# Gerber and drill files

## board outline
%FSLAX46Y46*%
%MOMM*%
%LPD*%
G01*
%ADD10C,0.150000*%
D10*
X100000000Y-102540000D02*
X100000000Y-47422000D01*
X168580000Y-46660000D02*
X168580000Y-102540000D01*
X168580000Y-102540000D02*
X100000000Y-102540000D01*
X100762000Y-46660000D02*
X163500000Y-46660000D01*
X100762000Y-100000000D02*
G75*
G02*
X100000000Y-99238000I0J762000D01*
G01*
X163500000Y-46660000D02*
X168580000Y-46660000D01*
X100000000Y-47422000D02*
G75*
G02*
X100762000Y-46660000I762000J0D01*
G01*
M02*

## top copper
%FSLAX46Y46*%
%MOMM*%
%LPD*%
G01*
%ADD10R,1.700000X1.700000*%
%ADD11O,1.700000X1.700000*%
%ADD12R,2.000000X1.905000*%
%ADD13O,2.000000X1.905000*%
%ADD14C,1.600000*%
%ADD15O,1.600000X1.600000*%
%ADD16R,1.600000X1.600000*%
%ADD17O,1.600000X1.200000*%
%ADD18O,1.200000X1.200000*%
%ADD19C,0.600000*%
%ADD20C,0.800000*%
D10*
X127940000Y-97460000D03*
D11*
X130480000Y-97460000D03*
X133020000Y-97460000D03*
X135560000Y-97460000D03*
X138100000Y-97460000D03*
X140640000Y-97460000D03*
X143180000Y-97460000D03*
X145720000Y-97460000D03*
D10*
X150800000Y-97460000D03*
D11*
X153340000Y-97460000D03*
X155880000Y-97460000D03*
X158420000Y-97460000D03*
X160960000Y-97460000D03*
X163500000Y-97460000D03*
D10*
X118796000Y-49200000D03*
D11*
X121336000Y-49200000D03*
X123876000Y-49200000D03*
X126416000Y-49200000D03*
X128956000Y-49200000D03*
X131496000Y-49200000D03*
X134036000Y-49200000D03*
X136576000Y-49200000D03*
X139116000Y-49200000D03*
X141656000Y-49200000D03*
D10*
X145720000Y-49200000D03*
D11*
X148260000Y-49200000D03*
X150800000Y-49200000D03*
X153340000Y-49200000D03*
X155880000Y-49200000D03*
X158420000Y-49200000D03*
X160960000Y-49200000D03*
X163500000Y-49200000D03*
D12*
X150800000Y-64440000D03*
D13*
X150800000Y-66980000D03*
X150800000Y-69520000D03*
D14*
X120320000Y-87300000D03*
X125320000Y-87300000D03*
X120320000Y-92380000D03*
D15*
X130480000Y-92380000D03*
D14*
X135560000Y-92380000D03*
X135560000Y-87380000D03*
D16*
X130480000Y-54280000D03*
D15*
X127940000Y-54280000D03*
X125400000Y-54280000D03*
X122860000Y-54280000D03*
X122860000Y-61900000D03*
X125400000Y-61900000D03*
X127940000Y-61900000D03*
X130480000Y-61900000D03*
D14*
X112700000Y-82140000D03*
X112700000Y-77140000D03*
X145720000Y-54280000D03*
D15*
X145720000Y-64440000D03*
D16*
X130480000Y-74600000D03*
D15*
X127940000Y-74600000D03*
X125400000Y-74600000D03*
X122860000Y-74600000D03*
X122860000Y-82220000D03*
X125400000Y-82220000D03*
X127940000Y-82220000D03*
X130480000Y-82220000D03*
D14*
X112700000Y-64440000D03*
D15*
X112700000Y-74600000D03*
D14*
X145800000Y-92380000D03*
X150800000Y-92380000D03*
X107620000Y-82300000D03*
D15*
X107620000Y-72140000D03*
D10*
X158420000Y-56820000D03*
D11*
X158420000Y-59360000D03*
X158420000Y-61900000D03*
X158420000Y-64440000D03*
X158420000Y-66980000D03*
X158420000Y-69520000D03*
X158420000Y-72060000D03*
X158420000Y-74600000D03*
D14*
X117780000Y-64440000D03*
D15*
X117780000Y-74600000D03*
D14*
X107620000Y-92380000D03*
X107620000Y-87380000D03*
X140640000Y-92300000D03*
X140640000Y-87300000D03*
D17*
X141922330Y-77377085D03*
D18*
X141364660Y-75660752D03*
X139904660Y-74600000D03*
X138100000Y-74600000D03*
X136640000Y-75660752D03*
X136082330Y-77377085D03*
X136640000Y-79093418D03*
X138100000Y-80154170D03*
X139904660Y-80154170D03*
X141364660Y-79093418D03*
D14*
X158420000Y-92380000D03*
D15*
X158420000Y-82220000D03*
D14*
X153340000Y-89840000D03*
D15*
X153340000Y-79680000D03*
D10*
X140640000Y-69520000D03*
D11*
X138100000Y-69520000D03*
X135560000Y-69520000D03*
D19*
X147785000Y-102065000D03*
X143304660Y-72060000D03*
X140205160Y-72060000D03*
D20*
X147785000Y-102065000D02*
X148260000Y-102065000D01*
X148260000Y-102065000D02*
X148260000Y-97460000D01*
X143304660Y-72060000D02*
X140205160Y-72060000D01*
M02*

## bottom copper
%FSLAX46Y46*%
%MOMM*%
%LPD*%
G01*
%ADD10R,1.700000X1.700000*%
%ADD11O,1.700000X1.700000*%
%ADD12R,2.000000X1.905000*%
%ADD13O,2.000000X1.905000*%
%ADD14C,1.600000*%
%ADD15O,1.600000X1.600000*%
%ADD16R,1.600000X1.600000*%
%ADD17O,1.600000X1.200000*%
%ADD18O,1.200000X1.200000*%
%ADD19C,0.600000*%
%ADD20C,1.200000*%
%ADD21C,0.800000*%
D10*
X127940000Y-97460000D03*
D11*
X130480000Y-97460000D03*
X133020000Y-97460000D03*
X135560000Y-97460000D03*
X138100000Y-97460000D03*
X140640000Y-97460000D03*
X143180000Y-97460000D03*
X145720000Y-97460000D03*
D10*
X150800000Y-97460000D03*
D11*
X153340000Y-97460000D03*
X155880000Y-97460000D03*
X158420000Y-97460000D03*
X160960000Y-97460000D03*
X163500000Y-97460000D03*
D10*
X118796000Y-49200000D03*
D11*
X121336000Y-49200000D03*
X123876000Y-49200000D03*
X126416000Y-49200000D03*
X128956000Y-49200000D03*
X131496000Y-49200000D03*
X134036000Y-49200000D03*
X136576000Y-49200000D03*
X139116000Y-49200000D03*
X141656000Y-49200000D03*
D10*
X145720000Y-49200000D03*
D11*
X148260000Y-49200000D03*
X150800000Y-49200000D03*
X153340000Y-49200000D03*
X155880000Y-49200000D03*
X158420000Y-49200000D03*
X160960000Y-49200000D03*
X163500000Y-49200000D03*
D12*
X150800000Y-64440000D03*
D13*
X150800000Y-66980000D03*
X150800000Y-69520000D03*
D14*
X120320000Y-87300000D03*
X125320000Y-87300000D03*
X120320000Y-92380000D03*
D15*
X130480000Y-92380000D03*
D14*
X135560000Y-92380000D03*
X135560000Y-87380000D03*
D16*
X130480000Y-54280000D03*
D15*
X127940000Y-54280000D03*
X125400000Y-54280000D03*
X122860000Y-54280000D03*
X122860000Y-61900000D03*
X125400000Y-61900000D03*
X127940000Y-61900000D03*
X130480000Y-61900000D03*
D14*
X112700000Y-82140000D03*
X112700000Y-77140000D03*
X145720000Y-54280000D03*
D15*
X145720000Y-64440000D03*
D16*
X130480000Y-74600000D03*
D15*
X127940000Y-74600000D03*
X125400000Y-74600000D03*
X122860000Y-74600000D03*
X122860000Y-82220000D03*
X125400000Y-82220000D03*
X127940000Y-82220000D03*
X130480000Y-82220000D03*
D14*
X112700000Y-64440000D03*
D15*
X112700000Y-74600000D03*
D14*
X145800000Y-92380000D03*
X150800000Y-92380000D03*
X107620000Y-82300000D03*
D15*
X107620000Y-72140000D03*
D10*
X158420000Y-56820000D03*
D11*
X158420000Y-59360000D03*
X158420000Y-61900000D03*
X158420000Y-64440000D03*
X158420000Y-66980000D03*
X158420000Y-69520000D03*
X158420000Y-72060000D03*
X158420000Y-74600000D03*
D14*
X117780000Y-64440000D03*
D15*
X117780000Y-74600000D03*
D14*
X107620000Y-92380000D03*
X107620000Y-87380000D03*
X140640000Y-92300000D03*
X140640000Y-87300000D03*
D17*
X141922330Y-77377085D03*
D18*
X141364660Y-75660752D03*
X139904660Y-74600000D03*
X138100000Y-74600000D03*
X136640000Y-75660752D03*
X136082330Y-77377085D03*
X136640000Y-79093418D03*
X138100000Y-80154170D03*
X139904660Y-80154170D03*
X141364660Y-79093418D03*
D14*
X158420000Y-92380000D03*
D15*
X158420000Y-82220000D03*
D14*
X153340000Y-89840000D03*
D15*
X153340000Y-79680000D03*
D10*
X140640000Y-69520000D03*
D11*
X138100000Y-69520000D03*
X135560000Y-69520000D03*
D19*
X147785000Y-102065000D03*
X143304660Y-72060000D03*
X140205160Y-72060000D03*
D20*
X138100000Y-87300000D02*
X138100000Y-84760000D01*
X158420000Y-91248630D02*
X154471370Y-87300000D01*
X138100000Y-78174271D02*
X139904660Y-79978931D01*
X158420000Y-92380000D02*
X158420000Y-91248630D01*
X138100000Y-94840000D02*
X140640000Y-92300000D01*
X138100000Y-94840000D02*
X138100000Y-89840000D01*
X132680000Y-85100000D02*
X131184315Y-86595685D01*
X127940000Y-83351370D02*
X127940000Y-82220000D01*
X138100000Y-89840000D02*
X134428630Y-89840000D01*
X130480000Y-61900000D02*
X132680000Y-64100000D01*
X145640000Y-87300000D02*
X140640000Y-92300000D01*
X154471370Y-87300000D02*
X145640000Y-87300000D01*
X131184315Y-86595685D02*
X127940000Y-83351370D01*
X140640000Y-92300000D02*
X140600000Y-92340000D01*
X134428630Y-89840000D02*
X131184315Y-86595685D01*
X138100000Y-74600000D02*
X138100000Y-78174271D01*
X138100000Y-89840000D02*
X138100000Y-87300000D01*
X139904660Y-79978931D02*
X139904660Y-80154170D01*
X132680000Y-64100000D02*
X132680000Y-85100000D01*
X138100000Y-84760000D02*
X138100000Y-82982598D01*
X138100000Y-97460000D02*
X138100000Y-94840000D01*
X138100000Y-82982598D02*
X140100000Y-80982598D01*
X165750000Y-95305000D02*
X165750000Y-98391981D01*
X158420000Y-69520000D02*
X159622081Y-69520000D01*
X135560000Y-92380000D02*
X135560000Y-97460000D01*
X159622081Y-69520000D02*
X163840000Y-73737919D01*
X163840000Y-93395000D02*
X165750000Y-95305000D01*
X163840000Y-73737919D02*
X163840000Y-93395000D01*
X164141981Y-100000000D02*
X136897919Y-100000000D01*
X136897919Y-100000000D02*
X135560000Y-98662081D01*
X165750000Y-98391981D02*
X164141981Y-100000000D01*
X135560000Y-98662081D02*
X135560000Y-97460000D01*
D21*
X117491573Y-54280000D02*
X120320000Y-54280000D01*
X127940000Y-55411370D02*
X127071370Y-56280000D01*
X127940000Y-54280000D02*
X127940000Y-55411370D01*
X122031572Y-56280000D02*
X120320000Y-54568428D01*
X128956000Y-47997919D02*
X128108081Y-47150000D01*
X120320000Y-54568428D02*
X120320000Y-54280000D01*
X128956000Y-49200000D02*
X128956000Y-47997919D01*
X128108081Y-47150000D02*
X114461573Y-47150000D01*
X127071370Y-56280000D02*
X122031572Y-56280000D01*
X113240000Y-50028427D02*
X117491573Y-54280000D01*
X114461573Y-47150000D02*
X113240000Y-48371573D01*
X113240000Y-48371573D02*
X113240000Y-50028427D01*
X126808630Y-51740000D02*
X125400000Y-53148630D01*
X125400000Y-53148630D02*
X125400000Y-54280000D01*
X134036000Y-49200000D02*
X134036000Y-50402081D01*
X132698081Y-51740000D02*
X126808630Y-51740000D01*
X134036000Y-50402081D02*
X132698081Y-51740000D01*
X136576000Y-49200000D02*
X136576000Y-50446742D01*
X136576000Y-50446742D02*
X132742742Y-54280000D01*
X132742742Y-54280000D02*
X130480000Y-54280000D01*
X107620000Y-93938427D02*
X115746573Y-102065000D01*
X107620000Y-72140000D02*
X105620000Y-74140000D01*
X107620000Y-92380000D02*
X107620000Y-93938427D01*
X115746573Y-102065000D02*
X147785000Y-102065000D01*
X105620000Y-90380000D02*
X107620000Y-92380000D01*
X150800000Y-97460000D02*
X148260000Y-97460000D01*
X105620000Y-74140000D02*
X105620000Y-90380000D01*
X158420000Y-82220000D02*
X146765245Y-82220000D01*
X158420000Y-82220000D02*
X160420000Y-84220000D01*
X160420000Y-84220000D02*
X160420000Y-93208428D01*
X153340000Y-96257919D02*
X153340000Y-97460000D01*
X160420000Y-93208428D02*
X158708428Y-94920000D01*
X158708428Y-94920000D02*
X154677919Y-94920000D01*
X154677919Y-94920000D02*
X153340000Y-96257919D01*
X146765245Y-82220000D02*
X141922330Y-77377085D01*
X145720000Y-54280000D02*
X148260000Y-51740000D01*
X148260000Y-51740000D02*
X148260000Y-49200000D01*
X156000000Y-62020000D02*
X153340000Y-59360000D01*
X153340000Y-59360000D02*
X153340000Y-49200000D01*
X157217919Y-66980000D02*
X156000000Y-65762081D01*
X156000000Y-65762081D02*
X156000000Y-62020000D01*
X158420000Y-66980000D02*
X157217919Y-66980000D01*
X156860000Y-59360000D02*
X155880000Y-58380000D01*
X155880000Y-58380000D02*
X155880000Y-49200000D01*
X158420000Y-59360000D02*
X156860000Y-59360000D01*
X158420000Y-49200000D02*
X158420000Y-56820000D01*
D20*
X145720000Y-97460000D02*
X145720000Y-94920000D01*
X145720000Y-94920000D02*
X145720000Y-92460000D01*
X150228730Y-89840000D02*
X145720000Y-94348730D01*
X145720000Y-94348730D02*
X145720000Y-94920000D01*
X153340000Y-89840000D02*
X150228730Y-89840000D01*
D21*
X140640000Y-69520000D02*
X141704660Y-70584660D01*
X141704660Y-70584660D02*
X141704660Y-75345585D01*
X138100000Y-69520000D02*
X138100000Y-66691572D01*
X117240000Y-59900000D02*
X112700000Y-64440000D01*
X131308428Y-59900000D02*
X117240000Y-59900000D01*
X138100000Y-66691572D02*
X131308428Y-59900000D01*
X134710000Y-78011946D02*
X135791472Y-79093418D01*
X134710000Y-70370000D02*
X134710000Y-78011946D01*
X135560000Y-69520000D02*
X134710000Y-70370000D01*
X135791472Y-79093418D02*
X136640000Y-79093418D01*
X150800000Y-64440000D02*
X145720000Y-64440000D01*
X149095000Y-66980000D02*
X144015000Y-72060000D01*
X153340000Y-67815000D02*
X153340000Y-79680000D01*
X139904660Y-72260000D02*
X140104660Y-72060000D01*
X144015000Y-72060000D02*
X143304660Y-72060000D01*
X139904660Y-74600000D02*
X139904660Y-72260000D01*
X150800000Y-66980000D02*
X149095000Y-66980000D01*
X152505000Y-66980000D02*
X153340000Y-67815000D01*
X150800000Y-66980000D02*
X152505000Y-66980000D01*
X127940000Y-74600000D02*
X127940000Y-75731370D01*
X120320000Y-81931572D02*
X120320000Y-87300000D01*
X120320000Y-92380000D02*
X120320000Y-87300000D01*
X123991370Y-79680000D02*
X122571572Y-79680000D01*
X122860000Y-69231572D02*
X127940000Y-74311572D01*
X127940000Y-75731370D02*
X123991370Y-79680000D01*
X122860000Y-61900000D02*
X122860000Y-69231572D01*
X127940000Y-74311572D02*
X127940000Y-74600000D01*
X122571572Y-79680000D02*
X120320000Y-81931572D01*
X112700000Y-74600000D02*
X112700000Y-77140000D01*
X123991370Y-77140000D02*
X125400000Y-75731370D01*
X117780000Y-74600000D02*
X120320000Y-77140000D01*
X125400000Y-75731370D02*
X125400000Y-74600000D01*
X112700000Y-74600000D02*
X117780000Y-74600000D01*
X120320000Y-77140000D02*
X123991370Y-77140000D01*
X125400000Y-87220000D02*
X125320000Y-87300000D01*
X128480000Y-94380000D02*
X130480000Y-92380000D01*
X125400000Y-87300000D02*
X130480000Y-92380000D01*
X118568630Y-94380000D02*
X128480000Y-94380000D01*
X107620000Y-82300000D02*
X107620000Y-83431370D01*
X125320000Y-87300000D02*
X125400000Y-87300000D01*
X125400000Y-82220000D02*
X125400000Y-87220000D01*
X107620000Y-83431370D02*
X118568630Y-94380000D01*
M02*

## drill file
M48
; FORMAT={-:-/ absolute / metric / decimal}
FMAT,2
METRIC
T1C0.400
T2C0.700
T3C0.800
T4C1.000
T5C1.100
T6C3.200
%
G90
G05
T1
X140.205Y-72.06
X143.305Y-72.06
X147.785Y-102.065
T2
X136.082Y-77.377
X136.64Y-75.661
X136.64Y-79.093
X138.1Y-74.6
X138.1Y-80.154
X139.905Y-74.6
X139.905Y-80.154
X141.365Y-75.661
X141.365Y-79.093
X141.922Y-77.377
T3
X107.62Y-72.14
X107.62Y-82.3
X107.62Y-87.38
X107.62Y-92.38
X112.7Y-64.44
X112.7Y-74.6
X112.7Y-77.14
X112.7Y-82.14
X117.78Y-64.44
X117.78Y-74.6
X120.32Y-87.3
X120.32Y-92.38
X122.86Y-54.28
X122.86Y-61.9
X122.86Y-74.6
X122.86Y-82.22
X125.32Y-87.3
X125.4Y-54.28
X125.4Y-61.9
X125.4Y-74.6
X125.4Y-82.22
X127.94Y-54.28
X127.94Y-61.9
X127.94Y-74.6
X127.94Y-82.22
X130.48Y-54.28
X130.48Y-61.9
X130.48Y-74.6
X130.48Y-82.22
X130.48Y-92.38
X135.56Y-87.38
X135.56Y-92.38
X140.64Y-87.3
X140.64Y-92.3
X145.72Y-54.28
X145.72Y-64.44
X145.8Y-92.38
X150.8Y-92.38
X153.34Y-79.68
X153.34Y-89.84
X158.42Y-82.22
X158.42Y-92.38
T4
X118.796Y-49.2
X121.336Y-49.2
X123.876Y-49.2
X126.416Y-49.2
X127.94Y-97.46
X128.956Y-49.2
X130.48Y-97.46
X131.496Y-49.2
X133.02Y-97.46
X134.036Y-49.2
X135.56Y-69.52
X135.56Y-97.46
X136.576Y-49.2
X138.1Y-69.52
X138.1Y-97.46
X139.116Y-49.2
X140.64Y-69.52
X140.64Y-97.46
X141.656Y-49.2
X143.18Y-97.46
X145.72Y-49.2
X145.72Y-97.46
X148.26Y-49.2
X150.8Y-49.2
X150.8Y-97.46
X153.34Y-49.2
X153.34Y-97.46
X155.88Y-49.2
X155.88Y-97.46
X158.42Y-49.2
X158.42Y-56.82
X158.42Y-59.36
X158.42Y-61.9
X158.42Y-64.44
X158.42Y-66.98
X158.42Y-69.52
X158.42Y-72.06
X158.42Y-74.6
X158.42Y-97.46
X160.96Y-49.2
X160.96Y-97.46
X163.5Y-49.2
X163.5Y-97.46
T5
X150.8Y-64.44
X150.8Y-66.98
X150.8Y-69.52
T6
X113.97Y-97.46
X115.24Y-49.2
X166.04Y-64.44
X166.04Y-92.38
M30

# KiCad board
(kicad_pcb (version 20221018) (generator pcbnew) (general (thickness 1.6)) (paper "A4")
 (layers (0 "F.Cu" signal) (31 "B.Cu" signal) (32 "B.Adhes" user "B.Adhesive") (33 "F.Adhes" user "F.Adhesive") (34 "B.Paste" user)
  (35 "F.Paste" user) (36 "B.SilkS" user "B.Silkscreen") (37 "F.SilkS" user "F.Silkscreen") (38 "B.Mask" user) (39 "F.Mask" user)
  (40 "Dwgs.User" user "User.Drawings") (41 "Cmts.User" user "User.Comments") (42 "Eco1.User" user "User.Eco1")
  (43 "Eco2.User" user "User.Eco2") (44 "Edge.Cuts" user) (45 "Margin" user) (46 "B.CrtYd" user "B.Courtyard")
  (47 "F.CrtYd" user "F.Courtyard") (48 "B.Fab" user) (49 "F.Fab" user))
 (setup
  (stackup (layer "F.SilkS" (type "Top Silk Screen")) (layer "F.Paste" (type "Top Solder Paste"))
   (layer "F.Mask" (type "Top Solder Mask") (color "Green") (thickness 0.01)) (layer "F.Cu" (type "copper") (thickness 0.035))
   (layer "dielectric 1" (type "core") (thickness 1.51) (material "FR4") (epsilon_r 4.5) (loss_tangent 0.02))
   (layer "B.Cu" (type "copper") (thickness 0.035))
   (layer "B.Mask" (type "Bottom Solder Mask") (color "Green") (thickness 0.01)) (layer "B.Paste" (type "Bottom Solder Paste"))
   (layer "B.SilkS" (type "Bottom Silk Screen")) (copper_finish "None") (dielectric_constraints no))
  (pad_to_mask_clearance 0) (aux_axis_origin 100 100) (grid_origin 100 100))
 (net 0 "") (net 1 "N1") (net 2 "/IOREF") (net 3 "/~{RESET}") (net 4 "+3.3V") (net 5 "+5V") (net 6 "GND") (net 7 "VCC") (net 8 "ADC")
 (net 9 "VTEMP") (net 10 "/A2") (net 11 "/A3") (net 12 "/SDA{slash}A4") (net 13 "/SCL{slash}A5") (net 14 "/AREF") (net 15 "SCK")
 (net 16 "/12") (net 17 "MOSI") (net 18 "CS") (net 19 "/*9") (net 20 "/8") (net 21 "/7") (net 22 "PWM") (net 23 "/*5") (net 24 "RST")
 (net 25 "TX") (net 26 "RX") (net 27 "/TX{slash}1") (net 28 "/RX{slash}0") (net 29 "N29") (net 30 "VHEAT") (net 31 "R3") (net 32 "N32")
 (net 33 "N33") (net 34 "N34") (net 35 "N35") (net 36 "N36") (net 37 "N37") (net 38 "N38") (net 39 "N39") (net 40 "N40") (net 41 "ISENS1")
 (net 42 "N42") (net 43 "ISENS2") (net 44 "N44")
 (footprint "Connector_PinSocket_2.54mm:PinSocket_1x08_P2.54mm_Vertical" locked (layer "F.Cu") (at 127.94 97.46 90)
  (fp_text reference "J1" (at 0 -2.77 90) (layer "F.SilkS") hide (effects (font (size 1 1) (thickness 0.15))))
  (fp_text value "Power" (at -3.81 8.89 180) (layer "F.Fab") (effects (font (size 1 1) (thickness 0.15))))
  (pad "1" thru_hole rect locked (at 0 0 90) (size 1.7 1.7) (drill 1) (layers "*.Cu" "*.Mask") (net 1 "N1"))
  (pad "2" thru_hole oval locked (at 0 2.54 90) (size 1.7 1.7) (drill 1) (layers "*.Cu" "*.Mask") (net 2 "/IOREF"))
  (pad "3" thru_hole oval locked (at 0 5.08 90) (size 1.7 1.7) (drill 1) (layers "*.Cu" "*.Mask") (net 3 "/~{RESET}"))
  (pad "4" thru_hole oval locked (at 0 7.62 90) (size 1.7 1.7) (drill 1) (layers "*.Cu" "*.Mask") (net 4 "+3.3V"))
  (pad "5" thru_hole oval locked (at 0 10.16 90) (size 1.7 1.7) (drill 1) (layers "*.Cu" "*.Mask") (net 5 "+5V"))
  (pad "6" thru_hole oval locked (at 0 12.7 90) (size 1.7 1.7) (drill 1) (layers "*.Cu" "*.Mask") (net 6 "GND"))
  (pad "7" thru_hole oval locked (at 0 15.24 90) (size 1.7 1.7) (drill 1) (layers "*.Cu" "*.Mask") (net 6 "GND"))
  (pad "8" thru_hole oval locked (at 0 17.78 90) (size 1.7 1.7) (drill 1) (layers "*.Cu" "*.Mask") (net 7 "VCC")))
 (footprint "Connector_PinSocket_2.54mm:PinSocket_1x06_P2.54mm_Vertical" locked (layer "F.Cu") (at 150.8 97.46 90)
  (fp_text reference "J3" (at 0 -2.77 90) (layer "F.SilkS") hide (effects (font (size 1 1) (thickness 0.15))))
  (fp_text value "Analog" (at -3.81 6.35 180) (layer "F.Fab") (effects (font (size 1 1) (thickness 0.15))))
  (pad "1" thru_hole rect locked (at 0 0 90) (size 1.7 1.7) (drill 1) (layers "*.Cu" "*.Mask") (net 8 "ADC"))
  (pad "2" thru_hole oval locked (at 0 2.54 90) (size 1.7 1.7) (drill 1) (layers "*.Cu" "*.Mask") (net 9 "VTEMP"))
  (pad "3" thru_hole oval locked (at 0 5.08 90) (size 1.7 1.7) (drill 1) (layers "*.Cu" "*.Mask") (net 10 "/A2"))
  (pad "4" thru_hole oval locked (at 0 7.62 90) (size 1.7 1.7) (drill 1) (layers "*.Cu" "*.Mask") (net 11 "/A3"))
  (pad "5" thru_hole oval locked (at 0 10.16 90) (size 1.7 1.7) (drill 1) (layers "*.Cu" "*.Mask") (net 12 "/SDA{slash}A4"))
  (pad "6" thru_hole oval locked (at 0 12.7 90) (size 1.7 1.7) (drill 1) (layers "*.Cu" "*.Mask") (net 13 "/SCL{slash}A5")))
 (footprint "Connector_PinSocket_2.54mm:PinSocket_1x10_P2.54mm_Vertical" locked (layer "F.Cu") (at 118.796 49.2 90)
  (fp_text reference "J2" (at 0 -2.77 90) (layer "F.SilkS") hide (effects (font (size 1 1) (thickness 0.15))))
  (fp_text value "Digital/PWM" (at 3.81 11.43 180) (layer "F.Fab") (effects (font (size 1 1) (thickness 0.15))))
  (pad "1" thru_hole rect locked (at 0 0 90) (size 1.7 1.7) (drill 1) (layers "*.Cu" "*.Mask") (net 13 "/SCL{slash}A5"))
  (pad "2" thru_hole oval locked (at 0 2.54 90) (size 1.7 1.7) (drill 1) (layers "*.Cu" "*.Mask") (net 12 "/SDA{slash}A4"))
  (pad "3" thru_hole oval locked (at 0 5.08 90) (size 1.7 1.7) (drill 1) (layers "*.Cu" "*.Mask") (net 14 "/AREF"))
  (pad "4" thru_hole oval locked (at 0 7.62 90) (size 1.7 1.7) (drill 1) (layers "*.Cu" "*.Mask") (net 6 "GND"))
  (pad "5" thru_hole oval locked (at 0 10.16 90) (size 1.7 1.7) (drill 1) (layers "*.Cu" "*.Mask") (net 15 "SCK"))
  (pad "6" thru_hole oval locked (at 0 12.7 90) (size 1.7 1.7) (drill 1) (layers "*.Cu" "*.Mask") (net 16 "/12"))
  (pad "7" thru_hole oval locked (at 0 15.24 90) (size 1.7 1.7) (drill 1) (layers "*.Cu" "*.Mask") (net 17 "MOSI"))
  (pad "8" thru_hole oval locked (at 0 17.78 90) (size 1.7 1.7) (drill 1) (layers "*.Cu" "*.Mask") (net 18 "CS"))
  (pad "9" thru_hole oval locked (at 0 20.32 90) (size 1.7 1.7) (drill 1) (layers "*.Cu" "*.Mask") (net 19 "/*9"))
  (pad "10" thru_hole oval locked (at 0 22.86 90) (size 1.7 1.7) (drill 1) (layers "*.Cu" "*.Mask") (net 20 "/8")))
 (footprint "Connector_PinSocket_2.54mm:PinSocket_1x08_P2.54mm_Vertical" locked (layer "F.Cu") (at 145.72 49.2 90)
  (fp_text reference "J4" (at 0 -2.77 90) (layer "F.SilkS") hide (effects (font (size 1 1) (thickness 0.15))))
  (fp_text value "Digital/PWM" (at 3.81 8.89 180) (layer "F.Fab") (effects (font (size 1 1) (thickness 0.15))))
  (pad "1" thru_hole rect locked (at 0 0 90) (size 1.7 1.7) (drill 1) (layers "*.Cu" "*.Mask") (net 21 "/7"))
  (pad "2" thru_hole oval locked (at 0 2.54 90) (size 1.7 1.7) (drill 1) (layers "*.Cu" "*.Mask") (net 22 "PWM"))
  (pad "3" thru_hole oval locked (at 0 5.08 90) (size 1.7 1.7) (drill 1) (layers "*.Cu" "*.Mask") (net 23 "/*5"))
  (pad "4" thru_hole oval locked (at 0 7.62 90) (size 1.7 1.7) (drill 1) (layers "*.Cu" "*.Mask") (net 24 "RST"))
  (pad "5" thru_hole oval locked (at 0 10.16 90) (size 1.7 1.7) (drill 1) (layers "*.Cu" "*.Mask") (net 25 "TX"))
  (pad "6" thru_hole oval locked (at 0 12.7 90) (size 1.7 1.7) (drill 1) (layers "*.Cu" "*.Mask") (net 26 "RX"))
  (pad "7" thru_hole oval locked (at 0 15.24 90) (size 1.7 1.7) (drill 1) (layers "*.Cu" "*.Mask") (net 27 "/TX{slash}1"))
  (pad "8" thru_hole oval locked (at 0 17.78 90) (size 1.7 1.7) (drill 1) (layers "*.Cu" "*.Mask") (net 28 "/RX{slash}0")))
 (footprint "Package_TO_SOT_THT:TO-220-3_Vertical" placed (layer "F.Cu") (at 150.8 64.44 -90)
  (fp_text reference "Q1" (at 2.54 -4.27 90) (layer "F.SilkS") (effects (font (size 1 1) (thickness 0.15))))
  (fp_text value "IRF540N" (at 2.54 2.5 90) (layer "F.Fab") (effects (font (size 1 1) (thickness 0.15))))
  (pad "1" thru_hole rect (at 0 0 270) (size 1.905 2) (drill 1.1) (layers "*.Cu" "*.Mask") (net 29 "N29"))
  (pad "2" thru_hole oval (at 2.54 0 270) (size 1.905 2) (drill 1.1) (layers "*.Cu" "*.Mask") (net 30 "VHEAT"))
  (pad "3" thru_hole oval (at 5.08 0 270) (size 1.905 2) (drill 1.1) (layers "*.Cu" "*.Mask") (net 6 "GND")))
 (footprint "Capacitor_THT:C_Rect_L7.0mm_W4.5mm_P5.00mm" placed (layer "F.Cu") (at 120.32 87.3)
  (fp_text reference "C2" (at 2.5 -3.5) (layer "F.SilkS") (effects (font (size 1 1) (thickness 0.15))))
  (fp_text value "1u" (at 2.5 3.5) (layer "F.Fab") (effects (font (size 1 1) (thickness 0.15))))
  (pad "1" thru_hole circle (at 0 0) (size 1.6 1.6) (drill 0.8) (layers "*.Cu" "*.Mask") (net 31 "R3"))
  (pad "2" thru_hole circle (at 5 0) (size 1.6 1.6) (drill 0.8) (layers "*.Cu" "*.Mask") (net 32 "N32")))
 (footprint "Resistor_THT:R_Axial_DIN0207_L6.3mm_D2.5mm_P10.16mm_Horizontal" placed (layer "F.Cu") (at 120.32 92.38)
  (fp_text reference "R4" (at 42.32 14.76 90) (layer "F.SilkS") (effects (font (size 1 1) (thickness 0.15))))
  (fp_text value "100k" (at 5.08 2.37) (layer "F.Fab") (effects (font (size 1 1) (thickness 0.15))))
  (pad "1" thru_hole circle (at 0 0) (size 1.6 1.6) (drill 0.8) (layers "*.Cu" "*.Mask") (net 31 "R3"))
  (pad "2" thru_hole oval (at 10.16 0) (size 1.6 1.6) (drill 0.8) (layers "*.Cu" "*.Mask") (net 32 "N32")))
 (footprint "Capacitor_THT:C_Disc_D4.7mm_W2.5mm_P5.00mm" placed (layer "F.Cu") (at 135.56 92.38 90)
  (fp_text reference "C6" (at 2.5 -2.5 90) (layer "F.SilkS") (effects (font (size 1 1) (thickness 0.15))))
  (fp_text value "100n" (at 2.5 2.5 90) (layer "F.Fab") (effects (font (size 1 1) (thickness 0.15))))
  (pad "1" thru_hole circle (at 0 0 90) (size 1.6 1.6) (drill 0.8) (layers "*.Cu" "*.Mask") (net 4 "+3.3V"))
  (pad "2" thru_hole circle (at 5 0 90) (size 1.6 1.6) (drill 0.8) (layers "*.Cu" "*.Mask") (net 6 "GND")))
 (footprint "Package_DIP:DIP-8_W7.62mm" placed (layer "F.Cu") (at 130.48 54.28 -90)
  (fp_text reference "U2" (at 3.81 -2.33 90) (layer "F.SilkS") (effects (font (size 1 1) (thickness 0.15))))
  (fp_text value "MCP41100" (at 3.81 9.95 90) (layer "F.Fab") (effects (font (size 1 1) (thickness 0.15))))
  (pad "1" thru_hole rect (at 0 0 270) (size 1.6 1.6) (drill 0.8) (layers "*.Cu" "*.Mask") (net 18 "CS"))
  (pad "2" thru_hole oval (at 0 2.54 270) (size 1.6 1.6) (drill 0.8) (layers "*.Cu" "*.Mask") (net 15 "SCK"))
  (pad "3" thru_hole oval (at 0 5.08 270) (size 1.6 1.6) (drill 0.8) (layers "*.Cu" "*.Mask") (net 17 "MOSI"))
  (pad "4" thru_hole oval (at 0 7.62 270) (size 1.6 1.6) (drill 0.8) (layers "*.Cu" "*.Mask") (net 6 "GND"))
  (pad "5" thru_hole oval (at 7.62 7.62 270) (size 1.6 1.6) (drill 0.8) (layers "*.Cu" "*.Mask") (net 31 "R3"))
  (pad "6" thru_hole oval (at 7.62 5.08 270) (size 1.6 1.6) (drill 0.8) (layers "*.Cu" "*.Mask") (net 6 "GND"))
  (pad "7" thru_hole oval (at 7.62 2.54 270) (size 1.6 1.6) (drill 0.8) (layers "*.Cu" "*.Mask") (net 6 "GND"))
  (pad "8" thru_hole oval (at 7.62 0 270) (size 1.6 1.6) (drill 0.8) (layers "*.Cu" "*.Mask") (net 5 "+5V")))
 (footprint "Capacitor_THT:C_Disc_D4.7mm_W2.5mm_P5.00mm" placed (layer "F.Cu") (at 112.7 82.14 90)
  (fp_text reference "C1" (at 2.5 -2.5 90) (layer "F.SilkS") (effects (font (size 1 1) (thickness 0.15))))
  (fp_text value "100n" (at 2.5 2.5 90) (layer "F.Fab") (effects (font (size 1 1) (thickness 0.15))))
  (pad "1" thru_hole circle (at 0 0 90) (size 1.6 1.6) (drill 0.8) (layers "*.Cu" "*.Mask") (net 6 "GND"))
  (pad "2" thru_hole circle (at 5 0 90) (size 1.6 1.6) (drill 0.8) (layers "*.Cu" "*.Mask") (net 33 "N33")))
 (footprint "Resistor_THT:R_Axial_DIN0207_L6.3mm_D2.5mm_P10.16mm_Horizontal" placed (layer "F.Cu") (at 145.72 54.28 -90)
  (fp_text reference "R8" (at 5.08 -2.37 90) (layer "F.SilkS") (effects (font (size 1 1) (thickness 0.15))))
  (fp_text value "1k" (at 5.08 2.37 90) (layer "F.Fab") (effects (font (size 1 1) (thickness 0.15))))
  (pad "1" thru_hole circle (at 0 0 270) (size 1.6 1.6) (drill 0.8) (layers "*.Cu" "*.Mask") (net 22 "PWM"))
  (pad "2" thru_hole oval (at 10.16 0 270) (size 1.6 1.6) (drill 0.8) (layers "*.Cu" "*.Mask") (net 29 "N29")))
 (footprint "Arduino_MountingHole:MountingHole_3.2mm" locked (layer "F.Cu") (at 115.24 49.2)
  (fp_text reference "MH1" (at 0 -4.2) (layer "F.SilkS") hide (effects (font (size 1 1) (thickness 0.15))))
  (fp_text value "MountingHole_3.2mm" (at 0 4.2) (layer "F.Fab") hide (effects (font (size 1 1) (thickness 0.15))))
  (pad "" np_thru_hole circle locked (at 0 0) (size 3.2 3.2) (drill 3.2) (layers "*.Cu" "*.Mask")))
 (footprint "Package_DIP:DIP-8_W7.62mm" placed (layer "F.Cu") (at 130.48 74.6 -90)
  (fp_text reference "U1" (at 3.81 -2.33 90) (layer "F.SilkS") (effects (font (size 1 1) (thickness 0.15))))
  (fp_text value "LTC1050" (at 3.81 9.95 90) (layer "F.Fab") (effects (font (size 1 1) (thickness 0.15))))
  (pad "1" thru_hole rect (at 0 0 270) (size 1.6 1.6) (drill 0.8) (layers "*.Cu" "*.Mask") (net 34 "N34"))
  (pad "2" thru_hole oval (at 0 2.54 270) (size 1.6 1.6) (drill 0.8) (layers "*.Cu" "*.Mask") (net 31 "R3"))
  (pad "3" thru_hole oval (at 0 5.08 270) (size 1.6 1.6) (drill 0.8) (layers "*.Cu" "*.Mask") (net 33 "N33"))
  (pad "4" thru_hole oval (at 0 7.62 270) (size 1.6 1.6) (drill 0.8) (layers "*.Cu" "*.Mask") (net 6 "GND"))
  (pad "5" thru_hole oval (at 7.62 7.62 270) (size 1.6 1.6) (drill 0.8) (layers "*.Cu" "*.Mask") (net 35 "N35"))
  (pad "6" thru_hole oval (at 7.62 5.08 270) (size 1.6 1.6) (drill 0.8) (layers "*.Cu" "*.Mask") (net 32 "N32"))
  (pad "7" thru_hole oval (at 7.62 2.54 270) (size 1.6 1.6) (drill 0.8) (layers "*.Cu" "*.Mask") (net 5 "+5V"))
  (pad "8" thru_hole oval (at 7.62 0 270) (size 1.6 1.6) (drill 0.8) (layers "*.Cu" "*.Mask") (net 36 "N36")))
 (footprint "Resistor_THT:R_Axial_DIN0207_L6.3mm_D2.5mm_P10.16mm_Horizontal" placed (layer "F.Cu") (at 112.7 64.44 -90)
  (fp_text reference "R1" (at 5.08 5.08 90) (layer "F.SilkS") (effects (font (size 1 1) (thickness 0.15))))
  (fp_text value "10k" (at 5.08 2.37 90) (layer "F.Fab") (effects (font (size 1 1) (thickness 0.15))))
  (pad "1" thru_hole circle (at 0 0 270) (size 1.6 1.6) (drill 0.8) (layers "*.Cu" "*.Mask") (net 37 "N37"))
  (pad "2" thru_hole oval (at 10.16 0 270) (size 1.6 1.6) (drill 0.8) (layers "*.Cu" "*.Mask") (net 33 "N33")))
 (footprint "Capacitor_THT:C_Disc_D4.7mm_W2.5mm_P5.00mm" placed (layer "F.Cu") (at 145.8 92.38)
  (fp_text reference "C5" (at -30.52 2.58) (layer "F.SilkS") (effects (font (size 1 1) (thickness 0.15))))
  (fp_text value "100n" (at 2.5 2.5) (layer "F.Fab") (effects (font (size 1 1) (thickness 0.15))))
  (pad "1" thru_hole circle (at 0 0) (size 1.6 1.6) (drill 0.8) (layers "*.Cu" "*.Mask") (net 7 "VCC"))
  (pad "2" thru_hole circle (at 5 0) (size 1.6 1.6) (drill 0.8) (layers "*.Cu" "*.Mask") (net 6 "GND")))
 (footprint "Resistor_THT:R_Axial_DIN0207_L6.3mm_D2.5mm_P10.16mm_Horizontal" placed (layer "F.Cu") (at 107.62 82.3 90)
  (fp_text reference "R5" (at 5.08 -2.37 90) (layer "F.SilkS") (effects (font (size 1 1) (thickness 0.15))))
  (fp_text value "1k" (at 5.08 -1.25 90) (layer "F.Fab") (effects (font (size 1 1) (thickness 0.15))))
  (pad "1" thru_hole circle (at 0 0 90) (size 1.6 1.6) (drill 0.8) (layers "*.Cu" "*.Mask") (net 32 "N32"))
  (pad "2" thru_hole oval (at 10.16 0 90) (size 1.6 1.6) (drill 0.8) (layers "*.Cu" "*.Mask") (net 8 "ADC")))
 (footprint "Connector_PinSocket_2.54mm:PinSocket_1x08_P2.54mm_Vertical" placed (layer "F.Cu") (at 158.42 56.82)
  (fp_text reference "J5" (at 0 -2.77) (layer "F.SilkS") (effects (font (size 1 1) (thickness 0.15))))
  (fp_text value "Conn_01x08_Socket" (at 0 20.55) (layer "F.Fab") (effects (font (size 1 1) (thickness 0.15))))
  (pad "1" thru_hole rect (at 0 0) (size 1.7 1.7) (drill 1) (layers "*.Cu" "*.Mask") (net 26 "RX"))
  (pad "2" thru_hole oval (at 0 2.54) (size 1.7 1.7) (drill 1) (layers "*.Cu" "*.Mask") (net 25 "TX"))
  (pad "3" thru_hole oval (at 0 5.08) (size 1.7 1.7) (drill 1) (layers "*.Cu" "*.Mask") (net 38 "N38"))
  (pad "4" thru_hole oval (at 0 7.62) (size 1.7 1.7) (drill 1) (layers "*.Cu" "*.Mask") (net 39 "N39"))
  (pad "5" thru_hole oval (at 0 10.16) (size 1.7 1.7) (drill 1) (layers "*.Cu" "*.Mask") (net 24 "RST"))
  (pad "6" thru_hole oval (at 0 12.7) (size 1.7 1.7) (drill 1) (layers "*.Cu" "*.Mask") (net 4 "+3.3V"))
  (pad "7" thru_hole oval (at 0 15.24) (size 1.7 1.7) (drill 1) (layers "*.Cu" "*.Mask") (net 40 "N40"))
  (pad "8" thru_hole oval (at 0 17.78) (size 1.7 1.7) (drill 1) (layers "*.Cu" "*.Mask") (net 6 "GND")))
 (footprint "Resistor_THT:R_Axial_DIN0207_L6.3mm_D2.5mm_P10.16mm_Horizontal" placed (layer "F.Cu") (at 117.78 64.44 -90)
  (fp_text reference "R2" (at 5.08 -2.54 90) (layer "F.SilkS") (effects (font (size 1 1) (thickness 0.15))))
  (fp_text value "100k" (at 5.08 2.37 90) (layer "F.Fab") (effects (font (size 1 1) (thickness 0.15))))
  (pad "1" thru_hole circle (at 0 0 270) (size 1.6 1.6) (drill 0.8) (layers "*.Cu" "*.Mask") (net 6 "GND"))
  (pad "2" thru_hole oval (at 10.16 0 270) (size 1.6 1.6) (drill 0.8) (layers "*.Cu" "*.Mask") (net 33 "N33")))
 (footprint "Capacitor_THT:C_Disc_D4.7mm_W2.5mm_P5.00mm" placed (layer "F.Cu") (at 107.62 92.38 90)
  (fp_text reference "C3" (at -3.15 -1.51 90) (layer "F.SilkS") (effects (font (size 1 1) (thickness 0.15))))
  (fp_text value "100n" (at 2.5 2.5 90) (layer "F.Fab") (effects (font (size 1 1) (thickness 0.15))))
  (pad "1" thru_hole circle (at 0 0 90) (size 1.6 1.6) (drill 0.8) (layers "*.Cu" "*.Mask") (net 8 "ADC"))
  (pad "2" thru_hole circle (at 5 0 90) (size 1.6 1.6) (drill 0.8) (layers "*.Cu" "*.Mask") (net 6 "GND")))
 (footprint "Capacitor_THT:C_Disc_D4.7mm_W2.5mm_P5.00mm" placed (layer "F.Cu") (at 140.64 92.3 90)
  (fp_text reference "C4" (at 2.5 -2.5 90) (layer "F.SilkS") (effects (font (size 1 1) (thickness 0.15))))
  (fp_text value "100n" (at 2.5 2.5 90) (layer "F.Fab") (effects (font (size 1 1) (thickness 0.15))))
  (pad "1" thru_hole circle (at 0 0 90) (size 1.6 1.6) (drill 0.8) (layers "*.Cu" "*.Mask") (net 5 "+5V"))
  (pad "2" thru_hole circle (at 5 0 90) (size 1.6 1.6) (drill 0.8) (layers "*.Cu" "*.Mask") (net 6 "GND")))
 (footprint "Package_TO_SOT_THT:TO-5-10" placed (layer "F.Cu") (at 141.92233 77.377085 180)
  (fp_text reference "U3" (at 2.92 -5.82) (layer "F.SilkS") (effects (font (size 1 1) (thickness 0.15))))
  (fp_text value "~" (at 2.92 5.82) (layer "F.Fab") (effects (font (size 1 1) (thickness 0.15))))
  (pad "1" thru_hole oval (at 0 0 180) (size 1.6 1.2) (drill 0.7) (layers "*.Cu" "*.Mask") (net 9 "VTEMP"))
  (pad "2" thru_hole oval (at 0.55767 1.716333 180) (size 1.2 1.2) (drill 0.7) (layers "*.Cu" "*.Mask") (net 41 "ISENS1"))
  (pad "3" thru_hole oval (at 2.01767 2.777085 180) (size 1.2 1.2) (drill 0.7) (layers "*.Cu" "*.Mask") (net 30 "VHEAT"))
  (pad "4" thru_hole oval (at 3.82233 2.777085 180) (size 1.2 1.2) (drill 0.7) (layers "*.Cu" "*.Mask") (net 5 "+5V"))
  (pad "5" thru_hole oval (at 5.28233 1.716333 180) (size 1.2 1.2) (drill 0.7) (layers "*.Cu" "*.Mask") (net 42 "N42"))
  (pad "6" thru_hole oval (at 5.84 0 180) (size 1.2 1.2) (drill 0.7) (layers "*.Cu" "*.Mask") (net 6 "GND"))
  (pad "7" thru_hole oval (at 5.28233 -1.716333 180) (size 1.2 1.2) (drill 0.7) (layers "*.Cu" "*.Mask") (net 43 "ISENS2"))
  (pad "8" thru_hole oval (at 3.82233 -2.777085 180) (size 1.2 1.2) (drill 0.7) (layers "*.Cu" "*.Mask") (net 6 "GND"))
  (pad "9" thru_hole oval (at 2.01767 -2.777085 180) (size 1.2 1.2) (drill 0.7) (layers "*.Cu" "*.Mask") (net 5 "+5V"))
  (pad "10" thru_hole oval (at 0.55767 -1.716333 180) (size 1.2 1.2) (drill 0.7) (layers "*.Cu" "*.Mask") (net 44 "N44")))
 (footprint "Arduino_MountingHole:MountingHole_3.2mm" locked (layer "F.Cu") (at 113.97 97.46)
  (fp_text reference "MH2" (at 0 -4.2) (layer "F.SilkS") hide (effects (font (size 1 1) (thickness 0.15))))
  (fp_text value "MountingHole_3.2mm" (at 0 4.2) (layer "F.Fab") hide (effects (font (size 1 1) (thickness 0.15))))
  (pad "" np_thru_hole circle locked (at 0 0) (size 3.2 3.2) (drill 3.2) (layers "*.Cu" "*.Mask")))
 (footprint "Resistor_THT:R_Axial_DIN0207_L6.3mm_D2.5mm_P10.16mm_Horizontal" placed (layer "F.Cu") (at 158.42 92.38 90)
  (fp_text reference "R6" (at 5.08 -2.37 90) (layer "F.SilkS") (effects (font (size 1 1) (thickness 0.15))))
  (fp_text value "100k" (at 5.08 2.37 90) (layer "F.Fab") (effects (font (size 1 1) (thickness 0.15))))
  (pad "1" thru_hole circle (at 0 0 90) (size 1.6 1.6) (drill 0.8) (layers "*.Cu" "*.Mask") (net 5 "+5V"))
  (pad "2" thru_hole oval (at 10.16 0 90) (size 1.6 1.6) (drill 0.8) (layers "*.Cu" "*.Mask") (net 9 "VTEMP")))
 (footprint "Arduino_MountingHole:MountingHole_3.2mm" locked (layer "F.Cu") (at 166.04 64.44)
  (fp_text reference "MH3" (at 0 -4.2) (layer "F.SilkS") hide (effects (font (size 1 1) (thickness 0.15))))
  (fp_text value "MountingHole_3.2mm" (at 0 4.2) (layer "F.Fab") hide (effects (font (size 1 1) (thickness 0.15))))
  (pad "" np_thru_hole circle locked (at 0 0) (size 3.2 3.2) (drill 3.2) (layers "*.Cu" "*.Mask")))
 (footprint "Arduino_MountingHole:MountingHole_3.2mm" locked (layer "F.Cu") (at 166.04 92.38)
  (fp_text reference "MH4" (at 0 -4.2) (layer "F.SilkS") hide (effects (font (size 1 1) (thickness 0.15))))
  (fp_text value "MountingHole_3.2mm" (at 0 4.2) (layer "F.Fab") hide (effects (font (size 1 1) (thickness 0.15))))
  (pad "" np_thru_hole circle locked (at 0 0) (size 3.2 3.2) (drill 3.2) (layers "*.Cu" "*.Mask")))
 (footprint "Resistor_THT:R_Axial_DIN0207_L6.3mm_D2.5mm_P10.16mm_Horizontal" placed (layer "F.Cu") (at 153.34 89.84 90)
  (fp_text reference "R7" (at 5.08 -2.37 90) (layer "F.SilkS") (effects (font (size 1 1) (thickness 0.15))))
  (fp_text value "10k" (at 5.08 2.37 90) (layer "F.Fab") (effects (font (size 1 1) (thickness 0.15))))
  (pad "1" thru_hole circle (at 0 0 90) (size 1.6 1.6) (drill 0.8) (layers "*.Cu" "*.Mask") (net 7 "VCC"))
  (pad "2" thru_hole oval (at 10.16 0 90) (size 1.6 1.6) (drill 0.8) (layers "*.Cu" "*.Mask") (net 30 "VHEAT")))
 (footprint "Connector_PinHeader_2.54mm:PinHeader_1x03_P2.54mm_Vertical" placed (layer "F.Cu") (at 140.64 69.52 -90)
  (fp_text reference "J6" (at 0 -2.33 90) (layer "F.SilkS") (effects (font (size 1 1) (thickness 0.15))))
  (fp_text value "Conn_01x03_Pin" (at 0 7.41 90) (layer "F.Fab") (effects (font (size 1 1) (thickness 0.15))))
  (pad "1" thru_hole rect (at 0 0 270) (size 1.7 1.7) (drill 1) (layers "*.Cu" "*.Mask") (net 41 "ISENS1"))
  (pad "2" thru_hole oval (at 0 2.54 270) (size 1.7 1.7) (drill 1) (layers "*.Cu" "*.Mask") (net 37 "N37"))
  (pad "3" thru_hole oval (at 0 5.08 270) (size 1.7 1.7) (drill 1) (layers "*.Cu" "*.Mask") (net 43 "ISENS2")))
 (gr_line (start 100 102.54) (end 100 47.422) (stroke (width 0.15) (type solid)) (layer "Edge.Cuts"))
 (gr_line (start 168.58 46.66) (end 168.58 102.54) (stroke (width 0.15) (type solid)) (layer "Edge.Cuts"))
 (gr_line (start 168.58 102.54) (end 100 102.54) (stroke (width 0.15) (type solid)) (layer "Edge.Cuts"))
 (gr_line (start 100.762 46.66) (end 163.5 46.66) (stroke (width 0.15) (type solid)) (layer "Edge.Cuts"))
 (gr_arc (start 100.762 100) (mid 100.223185 99.776815) (end 100 99.238) (stroke (width 0.15) (type solid)) (layer "Edge.Cuts"))
 (gr_line (start 163.5 46.66) (end 168.58 46.66) (stroke (width 0.15) (type solid)) (layer "Edge.Cuts"))
 (gr_arc (start 100 47.422) (mid 100.223185 46.883185) (end 100.762 46.66) (stroke (width 0.15) (type solid)) (layer "Edge.Cuts"))
 (segment (start 138.1 87.3) (end 138.1 84.76) (width 1.2) (layer "B.Cu") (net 5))
 (segment (start 158.42 91.24863) (end 154.47137 87.3) (width 1.2) (layer "B.Cu") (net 5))
 (segment (start 138.1 78.174271) (end 139.90466 79.978931) (width 1.2) (layer "B.Cu") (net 5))
 (segment (start 158.42 92.38) (end 158.42 91.24863) (width 1.2) (layer "B.Cu") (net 5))
 (segment (start 138.1 94.84) (end 140.64 92.3) (width 1.2) (layer "B.Cu") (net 5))
 (segment (start 138.1 94.84) (end 138.1 89.84) (width 1.2) (layer "B.Cu") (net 5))
 (segment (start 132.68 85.1) (end 131.184315 86.595685) (width 1.2) (layer "B.Cu") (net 5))
 (segment (start 127.94 83.35137) (end 127.94 82.22) (width 1.2) (layer "B.Cu") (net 5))
 (segment (start 138.1 89.84) (end 134.42863 89.84) (width 1.2) (layer "B.Cu") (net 5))
 (segment (start 130.48 61.9) (end 132.68 64.1) (width 1.2) (layer "B.Cu") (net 5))
 (segment (start 145.64 87.3) (end 140.64 92.3) (width 1.2) (layer "B.Cu") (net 5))
 (segment (start 154.47137 87.3) (end 145.64 87.3) (width 1.2) (layer "B.Cu") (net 5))
 (segment (start 131.184315 86.595685) (end 127.94 83.35137) (width 1.2) (layer "B.Cu") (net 5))
 (segment (start 140.64 92.3) (end 140.6 92.34) (width 1.2) (layer "B.Cu") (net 5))
 (segment (start 134.42863 89.84) (end 131.184315 86.595685) (width 1.2) (layer "B.Cu") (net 5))
 (segment (start 138.1 74.6) (end 138.1 78.174271) (width 1.2) (layer "B.Cu") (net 5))
 (segment (start 138.1 89.84) (end 138.1 87.3) (width 1.2) (layer "B.Cu") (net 5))
 (segment (start 139.90466 79.978931) (end 139.90466 80.15417) (width 1.2) (layer "B.Cu") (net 5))
 (segment (start 132.68 64.1) (end 132.68 85.1) (width 1.2) (layer "B.Cu") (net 5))
 (segment (start 138.1 84.76) (end 138.1 82.982598) (width 1.2) (layer "B.Cu") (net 5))
 (segment (start 138.1 97.46) (end 138.1 94.84) (width 1.2) (layer "B.Cu") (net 5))
 (segment (start 138.1 82.982598) (end 140.1 80.982598) (width 1.2) (layer "B.Cu") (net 5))
 (segment (start 165.75 95.305) (end 165.75 98.391981) (width 1.2) (layer "B.Cu") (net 4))
 (segment (start 158.42 69.52) (end 159.622081 69.52) (width 1.2) (layer "B.Cu") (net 4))
 (segment (start 135.56 92.38) (end 135.56 97.46) (width 1.2) (layer "B.Cu") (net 4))
 (segment (start 159.622081 69.52) (end 163.84 73.737919) (width 1.2) (layer "B.Cu") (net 4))
 (segment (start 163.84 93.395) (end 165.75 95.305) (width 1.2) (layer "B.Cu") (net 4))
 (segment (start 163.84 73.737919) (end 163.84 93.395) (width 1.2) (layer "B.Cu") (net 4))
 (segment (start 164.141981 100) (end 136.897919 100) (width 1.2) (layer "B.Cu") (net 4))
 (segment (start 136.897919 100) (end 135.56 98.662081) (width 1.2) (layer "B.Cu") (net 4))
 (segment (start 165.75 98.391981) (end 164.141981 100) (width 1.2) (layer "B.Cu") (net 4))
 (segment (start 135.56 98.662081) (end 135.56 97.46) (width 1.2) (layer "B.Cu") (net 4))
 (segment (start 117.491573 54.28) (end 120.32 54.28) (width 0.8) (layer "B.Cu") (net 15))
 (segment (start 127.94 55.41137) (end 127.07137 56.28) (width 0.8) (layer "B.Cu") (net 15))
 (segment (start 127.94 54.28) (end 127.94 55.41137) (width 0.8) (layer "B.Cu") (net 15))
 (segment (start 122.031572 56.28) (end 120.32 54.568428) (width 0.8) (layer "B.Cu") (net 15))
 (segment (start 128.956 47.997919) (end 128.108081 47.15) (width 0.8) (layer "B.Cu") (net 15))
 (segment (start 120.32 54.568428) (end 120.32 54.28) (width 0.8) (layer "B.Cu") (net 15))
 (segment (start 128.956 49.2) (end 128.956 47.997919) (width 0.8) (layer "B.Cu") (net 15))
 (segment (start 128.108081 47.15) (end 114.461573 47.15) (width 0.8) (layer "B.Cu") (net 15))
 (segment (start 127.07137 56.28) (end 122.031572 56.28) (width 0.8) (layer "B.Cu") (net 15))
 (segment (start 113.24 50.028427) (end 117.491573 54.28) (width 0.8) (layer "B.Cu") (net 15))
 (segment (start 114.461573 47.15) (end 113.24 48.371573) (width 0.8) (layer "B.Cu") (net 15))
 (segment (start 113.24 48.371573) (end 113.24 50.028427) (width 0.8) (layer "B.Cu") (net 15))
 (segment (start 126.80863 51.74) (end 125.4 53.14863) (width 0.8) (layer "B.Cu") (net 17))
 (segment (start 125.4 53.14863) (end 125.4 54.28) (width 0.8) (layer "B.Cu") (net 17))
 (segment (start 134.036 49.2) (end 134.036 50.402081) (width 0.8) (layer "B.Cu") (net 17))
 (segment (start 132.698081 51.74) (end 126.80863 51.74) (width 0.8) (layer "B.Cu") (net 17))
 (segment (start 134.036 50.402081) (end 132.698081 51.74) (width 0.8) (layer "B.Cu") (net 17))
 (segment (start 136.576 49.2) (end 136.576 50.446742) (width 0.8) (layer "B.Cu") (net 18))
 (segment (start 136.576 50.446742) (end 132.742742 54.28) (width 0.8) (layer "B.Cu") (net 18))
 (segment (start 132.742742 54.28) (end 130.48 54.28) (width 0.8) (layer "B.Cu") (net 18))
 (segment (start 147.785 102.065) (end 148.26 102.065) (width 0.8) (layer "F.Cu") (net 8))
 (segment (start 148.26 102.065) (end 148.26 97.46) (width 0.8) (layer "F.Cu") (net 8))
 (via (at 147.785 102.065) (size 0.6) (drill 0.4) (layers "F.Cu" "B.Cu") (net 8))
 (segment (start 107.62 93.938427) (end 115.746573 102.065) (width 0.8) (layer "B.Cu") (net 8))
 (segment (start 107.62 72.14) (end 105.62 74.14) (width 0.8) (layer "B.Cu") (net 8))
 (segment (start 107.62 92.38) (end 107.62 93.938427) (width 0.8) (layer "B.Cu") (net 8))
 (segment (start 115.746573 102.065) (end 147.785 102.065) (width 0.8) (layer "B.Cu") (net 8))
 (segment (start 105.62 90.38) (end 107.62 92.38) (width 0.8) (layer "B.Cu") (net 8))
 (segment (start 150.8 97.46) (end 148.26 97.46) (width 0.8) (layer "B.Cu") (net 8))
 (segment (start 105.62 74.14) (end 105.62 90.38) (width 0.8) (layer "B.Cu") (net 8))
 (segment (start 158.42 82.22) (end 146.765245 82.22) (width 0.8) (layer "B.Cu") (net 9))
 (segment (start 158.42 82.22) (end 160.42 84.22) (width 0.8) (layer "B.Cu") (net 9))
 (segment (start 160.42 84.22) (end 160.42 93.208428) (width 0.8) (layer "B.Cu") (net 9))
 (segment (start 153.34 96.257919) (end 153.34 97.46) (width 0.8) (layer "B.Cu") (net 9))
 (segment (start 160.42 93.208428) (end 158.708428 94.92) (width 0.8) (layer "B.Cu") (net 9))
 (segment (start 158.708428 94.92) (end 154.677919 94.92) (width 0.8) (layer "B.Cu") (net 9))
 (segment (start 154.677919 94.92) (end 153.34 96.257919) (width 0.8) (layer "B.Cu") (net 9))
 (segment (start 146.765245 82.22) (end 141.92233 77.377085) (width 0.8) (layer "B.Cu") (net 9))
 (segment (start 145.72 54.28) (end 148.26 51.74) (width 0.8) (layer "B.Cu") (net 22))
 (segment (start 148.26 51.74) (end 148.26 49.2) (width 0.8) (layer "B.Cu") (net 22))
 (segment (start 156 62.02) (end 153.34 59.36) (width 0.8) (layer "B.Cu") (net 24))
 (segment (start 153.34 59.36) (end 153.34 49.2) (width 0.8) (layer "B.Cu") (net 24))
 (segment (start 157.217919 66.98) (end 156 65.762081) (width 0.8) (layer "B.Cu") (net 24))
 (segment (start 156 65.762081) (end 156 62.02) (width 0.8) (layer "B.Cu") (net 24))
 (segment (start 158.42 66.98) (end 157.217919 66.98) (width 0.8) (layer "B.Cu") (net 24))
 (segment (start 156.86 59.36) (end 155.88 58.38) (width 0.8) (layer "B.Cu") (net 25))
 (segment (start 155.88 58.38) (end 155.88 49.2) (width 0.8) (layer "B.Cu") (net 25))
 (segment (start 158.42 59.36) (end 156.86 59.36) (width 0.8) (layer "B.Cu") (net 25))
 (segment (start 158.42 49.2) (end 158.42 56.82) (width 0.8) (layer "B.Cu") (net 26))
 (segment (start 145.72 97.46) (end 145.72 94.92) (width 1.2) (layer "B.Cu") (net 7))
 (segment (start 145.72 94.92) (end 145.72 92.46) (width 1.2) (layer "B.Cu") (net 7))
 (segment (start 150.22873 89.84) (end 145.72 94.34873) (width 1.2) (layer "B.Cu") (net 7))
 (segment (start 145.72 94.34873) (end 145.72 94.92) (width 1.2) (layer "B.Cu") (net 7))
 (segment (start 153.34 89.84) (end 150.22873 89.84) (width 1.2) (layer "B.Cu") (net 7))
 (segment (start 140.64 69.52) (end 141.70466 70.58466) (width 0.8) (layer "B.Cu") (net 41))
 (segment (start 141.70466 70.58466) (end 141.70466 75.345585) (width 0.8) (layer "B.Cu") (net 41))
 (segment (start 138.1 69.52) (end 138.1 66.691572) (width 0.8) (layer "B.Cu") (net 37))
 (segment (start 117.24 59.9) (end 112.7 64.44) (width 0.8) (layer "B.Cu") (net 37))
 (segment (start 131.308428 59.9) (end 117.24 59.9) (width 0.8) (layer "B.Cu") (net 37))
 (segment (start 138.1 66.691572) (end 131.308428 59.9) (width 0.8) (layer "B.Cu") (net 37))
 (segment (start 134.71 78.011946) (end 135.791472 79.093418) (width 0.8) (layer "B.Cu") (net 43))
 (segment (start 134.71 70.37) (end 134.71 78.011946) (width 0.8) (layer "B.Cu") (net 43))
 (segment (start 135.56 69.52) (end 134.71 70.37) (width 0.8) (layer "B.Cu") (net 43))
 (segment (start 135.791472 79.093418) (end 136.64 79.093418) (width 0.8) (layer "B.Cu") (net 43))
 (segment (start 150.8 64.44) (end 145.72 64.44) (width 0.8) (layer "B.Cu") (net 29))
 (segment (start 143.30466 72.06) (end 140.20516 72.06) (width 0.8) (layer "F.Cu") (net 30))
 (via (at 143.30466 72.06) (size 0.6) (drill 0.4) (layers "F.Cu" "B.Cu") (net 30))
 (via (at 140.20516 72.06) (size 0.6) (drill 0.4) (layers "F.Cu" "B.Cu") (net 30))
 (segment (start 149.095 66.98) (end 144.015 72.06) (width 0.8) (layer "B.Cu") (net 30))
 (segment (start 153.34 67.815) (end 153.34 79.68) (width 0.8) (layer "B.Cu") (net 30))
 (segment (start 139.90466 72.26) (end 140.10466 72.06) (width 0.8) (layer "B.Cu") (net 30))
 (segment (start 144.015 72.06) (end 143.30466 72.06) (width 0.8) (layer "B.Cu") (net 30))
 (segment (start 139.90466 74.6) (end 139.90466 72.26) (width 0.8) (layer "B.Cu") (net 30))
 (segment (start 150.8 66.98) (end 149.095 66.98) (width 0.8) (layer "B.Cu") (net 30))
 (segment (start 152.505 66.98) (end 153.34 67.815) (width 0.8) (layer "B.Cu") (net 30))
 (segment (start 150.8 66.98) (end 152.505 66.98) (width 0.8) (layer "B.Cu") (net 30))
 (segment (start 127.94 74.6) (end 127.94 75.73137) (width 0.8) (layer "B.Cu") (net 31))
 (segment (start 120.32 81.931572) (end 120.32 87.3) (width 0.8) (layer "B.Cu") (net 31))
 (segment (start 120.32 92.38) (end 120.32 87.3) (width 0.8) (layer "B.Cu") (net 31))
 (segment (start 123.99137 79.68) (end 122.571572 79.68) (width 0.8) (layer "B.Cu") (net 31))
 (segment (start 122.86 69.231572) (end 127.94 74.311572) (width 0.8) (layer "B.Cu") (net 31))
 (segment (start 127.94 75.73137) (end 123.99137 79.68) (width 0.8) (layer "B.Cu") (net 31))
 (segment (start 122.86 61.9) (end 122.86 69.231572) (width 0.8) (layer "B.Cu") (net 31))
 (segment (start 127.94 74.311572) (end 127.94 74.6) (width 0.8) (layer "B.Cu") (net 31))
 (segment (start 122.571572 79.68) (end 120.32 81.931572) (width 0.8) (layer "B.Cu") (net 31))
 (segment (start 112.7 74.6) (end 112.7 77.14) (width 0.8) (layer "B.Cu") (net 33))
 (segment (start 123.99137 77.14) (end 125.4 75.73137) (width 0.8) (layer "B.Cu") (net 33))
 (segment (start 117.78 74.6) (end 120.32 77.14) (width 0.8) (layer "B.Cu") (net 33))
 (segment (start 125.4 75.73137) (end 125.4 74.6) (width 0.8) (layer "B.Cu") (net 33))
 (segment (start 112.7 74.6) (end 117.78 74.6) (width 0.8) (layer "B.Cu") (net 33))
 (segment (start 120.32 77.14) (end 123.99137 77.14) (width 0.8) (layer "B.Cu") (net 33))
 (segment (start 125.4 87.22) (end 125.32 87.3) (width 0.8) (layer "B.Cu") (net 32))
 (segment (start 128.48 94.38) (end 130.48 92.38) (width 0.8) (layer "B.Cu") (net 32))
 (segment (start 125.4 87.3) (end 130.48 92.38) (width 0.8) (layer "B.Cu") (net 32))
 (segment (start 118.56863 94.38) (end 128.48 94.38) (width 0.8) (layer "B.Cu") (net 32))
 (segment (start 107.62 82.3) (end 107.62 83.43137) (width 0.8) (layer "B.Cu") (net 32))
 (segment (start 125.32 87.3) (end 125.4 87.3) (width 0.8) (layer "B.Cu") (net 32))
 (segment (start 125.4 82.22) (end 125.4 87.22) (width 0.8) (layer "B.Cu") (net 32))
 (segment (start 107.62 83.43137) (end 118.56863 94.38) (width 0.8) (layer "B.Cu") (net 32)))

